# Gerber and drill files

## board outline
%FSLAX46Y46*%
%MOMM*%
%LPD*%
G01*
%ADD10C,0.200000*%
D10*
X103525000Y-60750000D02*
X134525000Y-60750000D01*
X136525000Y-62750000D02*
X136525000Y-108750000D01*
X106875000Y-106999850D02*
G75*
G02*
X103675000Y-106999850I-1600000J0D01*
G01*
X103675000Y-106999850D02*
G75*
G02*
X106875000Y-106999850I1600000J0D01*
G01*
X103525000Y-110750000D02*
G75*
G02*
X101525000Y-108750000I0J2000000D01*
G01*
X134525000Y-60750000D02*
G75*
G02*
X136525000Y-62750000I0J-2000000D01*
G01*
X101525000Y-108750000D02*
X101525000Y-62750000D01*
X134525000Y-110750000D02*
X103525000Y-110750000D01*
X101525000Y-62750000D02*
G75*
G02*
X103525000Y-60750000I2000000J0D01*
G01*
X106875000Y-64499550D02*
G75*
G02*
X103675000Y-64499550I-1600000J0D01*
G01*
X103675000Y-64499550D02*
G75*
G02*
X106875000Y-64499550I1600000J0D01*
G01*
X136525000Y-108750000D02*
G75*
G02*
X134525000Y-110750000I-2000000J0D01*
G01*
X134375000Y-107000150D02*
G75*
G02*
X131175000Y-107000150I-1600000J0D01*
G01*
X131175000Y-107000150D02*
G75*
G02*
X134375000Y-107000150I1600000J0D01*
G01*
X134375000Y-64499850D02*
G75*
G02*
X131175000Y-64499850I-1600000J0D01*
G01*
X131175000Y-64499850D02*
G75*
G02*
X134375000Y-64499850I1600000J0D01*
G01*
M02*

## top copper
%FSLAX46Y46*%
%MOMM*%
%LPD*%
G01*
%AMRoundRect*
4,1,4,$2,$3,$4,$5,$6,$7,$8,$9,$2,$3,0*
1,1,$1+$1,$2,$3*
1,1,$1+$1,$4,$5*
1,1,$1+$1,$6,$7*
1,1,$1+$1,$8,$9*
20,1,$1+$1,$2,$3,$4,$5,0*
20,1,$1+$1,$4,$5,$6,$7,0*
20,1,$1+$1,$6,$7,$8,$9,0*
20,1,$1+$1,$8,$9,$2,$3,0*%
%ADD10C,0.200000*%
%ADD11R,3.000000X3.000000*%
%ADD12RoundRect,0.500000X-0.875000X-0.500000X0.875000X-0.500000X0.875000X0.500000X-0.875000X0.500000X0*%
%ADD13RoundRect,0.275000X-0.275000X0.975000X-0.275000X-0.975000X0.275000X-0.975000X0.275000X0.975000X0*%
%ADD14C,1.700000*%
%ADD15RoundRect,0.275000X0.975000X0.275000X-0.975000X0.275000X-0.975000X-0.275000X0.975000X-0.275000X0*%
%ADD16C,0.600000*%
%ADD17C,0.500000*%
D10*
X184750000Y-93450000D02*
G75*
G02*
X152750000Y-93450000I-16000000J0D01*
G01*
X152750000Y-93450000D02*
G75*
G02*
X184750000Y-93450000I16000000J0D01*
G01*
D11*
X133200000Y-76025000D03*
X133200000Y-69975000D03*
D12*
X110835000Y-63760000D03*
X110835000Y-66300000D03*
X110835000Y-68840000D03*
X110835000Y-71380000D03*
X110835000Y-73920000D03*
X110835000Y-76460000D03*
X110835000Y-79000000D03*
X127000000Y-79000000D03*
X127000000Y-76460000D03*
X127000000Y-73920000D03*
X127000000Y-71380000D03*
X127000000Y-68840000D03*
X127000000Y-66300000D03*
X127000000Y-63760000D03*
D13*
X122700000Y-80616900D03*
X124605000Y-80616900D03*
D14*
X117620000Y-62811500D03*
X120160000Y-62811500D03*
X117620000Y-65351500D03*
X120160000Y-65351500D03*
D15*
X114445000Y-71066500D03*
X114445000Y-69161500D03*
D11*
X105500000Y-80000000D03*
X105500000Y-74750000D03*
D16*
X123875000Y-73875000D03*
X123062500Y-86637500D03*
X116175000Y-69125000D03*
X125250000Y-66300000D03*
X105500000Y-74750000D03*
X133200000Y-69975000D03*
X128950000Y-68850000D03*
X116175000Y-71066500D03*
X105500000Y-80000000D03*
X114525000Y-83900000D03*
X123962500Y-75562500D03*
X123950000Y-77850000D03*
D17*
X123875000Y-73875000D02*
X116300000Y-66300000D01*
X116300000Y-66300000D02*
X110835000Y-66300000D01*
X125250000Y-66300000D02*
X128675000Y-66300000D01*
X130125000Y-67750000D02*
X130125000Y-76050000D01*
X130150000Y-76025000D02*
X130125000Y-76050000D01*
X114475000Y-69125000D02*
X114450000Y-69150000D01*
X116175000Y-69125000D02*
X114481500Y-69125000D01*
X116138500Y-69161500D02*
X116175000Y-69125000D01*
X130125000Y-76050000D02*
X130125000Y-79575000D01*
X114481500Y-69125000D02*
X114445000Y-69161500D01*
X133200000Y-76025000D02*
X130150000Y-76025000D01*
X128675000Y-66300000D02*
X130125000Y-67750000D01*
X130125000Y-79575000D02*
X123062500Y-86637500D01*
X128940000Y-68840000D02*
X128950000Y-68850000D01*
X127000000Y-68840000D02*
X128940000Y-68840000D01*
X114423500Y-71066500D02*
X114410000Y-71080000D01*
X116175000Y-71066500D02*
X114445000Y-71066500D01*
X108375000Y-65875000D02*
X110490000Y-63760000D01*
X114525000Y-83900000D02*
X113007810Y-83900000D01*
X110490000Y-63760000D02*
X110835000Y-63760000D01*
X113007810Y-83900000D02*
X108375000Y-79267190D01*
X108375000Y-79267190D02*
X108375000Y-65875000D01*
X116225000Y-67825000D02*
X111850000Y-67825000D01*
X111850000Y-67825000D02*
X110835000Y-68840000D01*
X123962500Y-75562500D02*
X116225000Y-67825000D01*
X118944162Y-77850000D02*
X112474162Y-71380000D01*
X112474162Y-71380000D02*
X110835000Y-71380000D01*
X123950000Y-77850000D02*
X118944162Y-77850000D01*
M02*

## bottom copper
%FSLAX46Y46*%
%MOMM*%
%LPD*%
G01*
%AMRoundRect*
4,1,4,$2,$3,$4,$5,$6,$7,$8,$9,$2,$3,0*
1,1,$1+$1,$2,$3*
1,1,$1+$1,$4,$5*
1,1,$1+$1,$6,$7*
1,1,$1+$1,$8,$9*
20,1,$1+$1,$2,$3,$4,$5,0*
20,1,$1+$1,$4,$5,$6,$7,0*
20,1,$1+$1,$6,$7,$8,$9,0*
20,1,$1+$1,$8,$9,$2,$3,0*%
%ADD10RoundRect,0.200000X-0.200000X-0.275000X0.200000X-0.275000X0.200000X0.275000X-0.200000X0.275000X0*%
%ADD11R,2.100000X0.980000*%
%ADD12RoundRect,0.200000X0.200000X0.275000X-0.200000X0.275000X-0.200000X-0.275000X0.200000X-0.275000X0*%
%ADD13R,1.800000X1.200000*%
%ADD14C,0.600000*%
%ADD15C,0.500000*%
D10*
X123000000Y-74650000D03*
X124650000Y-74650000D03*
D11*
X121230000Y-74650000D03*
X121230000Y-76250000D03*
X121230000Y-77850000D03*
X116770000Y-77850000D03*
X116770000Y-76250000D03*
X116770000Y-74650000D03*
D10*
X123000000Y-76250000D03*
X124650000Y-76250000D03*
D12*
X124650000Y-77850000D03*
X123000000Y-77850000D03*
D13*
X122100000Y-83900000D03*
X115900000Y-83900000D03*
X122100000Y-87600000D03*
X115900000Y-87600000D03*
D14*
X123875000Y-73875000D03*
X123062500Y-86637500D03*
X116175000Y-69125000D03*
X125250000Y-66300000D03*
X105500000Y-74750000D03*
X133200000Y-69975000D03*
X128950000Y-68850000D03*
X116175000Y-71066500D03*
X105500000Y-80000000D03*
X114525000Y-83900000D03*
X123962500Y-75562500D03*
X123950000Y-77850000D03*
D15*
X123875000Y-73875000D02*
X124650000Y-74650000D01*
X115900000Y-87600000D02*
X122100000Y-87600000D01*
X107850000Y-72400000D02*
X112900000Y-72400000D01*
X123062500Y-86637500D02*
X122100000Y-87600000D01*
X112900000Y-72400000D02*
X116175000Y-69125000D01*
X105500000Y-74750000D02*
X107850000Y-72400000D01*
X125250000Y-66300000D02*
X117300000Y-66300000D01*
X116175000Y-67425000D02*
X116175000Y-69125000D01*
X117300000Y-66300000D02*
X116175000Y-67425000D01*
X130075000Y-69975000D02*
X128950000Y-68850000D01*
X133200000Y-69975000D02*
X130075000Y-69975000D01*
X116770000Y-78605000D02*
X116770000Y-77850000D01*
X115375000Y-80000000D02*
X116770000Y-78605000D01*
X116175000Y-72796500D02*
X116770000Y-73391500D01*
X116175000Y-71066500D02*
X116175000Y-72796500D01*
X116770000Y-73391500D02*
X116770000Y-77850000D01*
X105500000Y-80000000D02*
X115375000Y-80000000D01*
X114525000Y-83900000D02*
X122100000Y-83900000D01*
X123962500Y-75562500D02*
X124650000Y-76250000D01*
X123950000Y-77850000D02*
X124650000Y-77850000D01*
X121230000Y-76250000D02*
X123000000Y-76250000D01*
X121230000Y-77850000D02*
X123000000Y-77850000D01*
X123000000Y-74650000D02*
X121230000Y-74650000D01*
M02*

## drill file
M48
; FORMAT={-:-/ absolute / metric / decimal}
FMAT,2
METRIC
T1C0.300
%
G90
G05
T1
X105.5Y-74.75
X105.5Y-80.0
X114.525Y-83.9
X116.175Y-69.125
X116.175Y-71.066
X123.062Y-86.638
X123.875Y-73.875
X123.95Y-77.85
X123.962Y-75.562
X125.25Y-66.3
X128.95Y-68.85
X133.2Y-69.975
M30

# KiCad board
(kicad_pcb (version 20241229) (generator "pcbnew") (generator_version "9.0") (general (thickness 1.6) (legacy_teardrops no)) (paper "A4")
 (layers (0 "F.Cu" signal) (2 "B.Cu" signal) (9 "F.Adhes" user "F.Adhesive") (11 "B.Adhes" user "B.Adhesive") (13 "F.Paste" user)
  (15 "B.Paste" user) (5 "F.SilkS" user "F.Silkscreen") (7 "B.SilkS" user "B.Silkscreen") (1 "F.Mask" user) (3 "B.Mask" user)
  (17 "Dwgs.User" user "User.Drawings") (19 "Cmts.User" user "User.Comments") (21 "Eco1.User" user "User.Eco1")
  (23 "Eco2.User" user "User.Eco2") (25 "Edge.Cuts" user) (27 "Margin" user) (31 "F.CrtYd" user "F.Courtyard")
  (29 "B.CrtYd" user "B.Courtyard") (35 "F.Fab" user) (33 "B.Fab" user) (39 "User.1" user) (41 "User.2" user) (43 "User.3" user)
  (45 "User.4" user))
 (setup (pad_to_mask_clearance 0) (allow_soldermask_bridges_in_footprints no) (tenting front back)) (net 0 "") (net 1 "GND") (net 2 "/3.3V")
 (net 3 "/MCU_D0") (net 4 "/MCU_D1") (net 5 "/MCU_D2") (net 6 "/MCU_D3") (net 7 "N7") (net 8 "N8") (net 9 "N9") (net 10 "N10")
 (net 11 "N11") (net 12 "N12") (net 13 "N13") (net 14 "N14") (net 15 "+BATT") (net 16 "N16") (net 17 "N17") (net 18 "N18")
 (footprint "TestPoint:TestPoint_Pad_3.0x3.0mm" (layer "F.Cu") (at 133.2 76.025)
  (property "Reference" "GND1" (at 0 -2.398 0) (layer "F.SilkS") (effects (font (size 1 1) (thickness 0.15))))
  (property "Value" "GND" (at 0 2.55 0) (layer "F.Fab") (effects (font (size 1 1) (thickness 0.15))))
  (pad "1" smd rect (at 0 0) (size 3 3) (layers "F.Cu" "F.Mask") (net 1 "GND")))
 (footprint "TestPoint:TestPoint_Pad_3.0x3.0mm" (layer "F.Cu") (at 133.2 69.975)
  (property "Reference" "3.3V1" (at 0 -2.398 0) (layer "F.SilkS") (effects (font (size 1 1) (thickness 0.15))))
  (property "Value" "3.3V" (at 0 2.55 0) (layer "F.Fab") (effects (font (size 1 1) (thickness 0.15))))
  (pad "1" smd rect (at 0 0) (size 3 3) (layers "F.Cu" "F.Mask") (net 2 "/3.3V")))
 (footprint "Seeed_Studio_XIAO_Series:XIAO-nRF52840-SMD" (layer "F.Cu") (at 110 81.88)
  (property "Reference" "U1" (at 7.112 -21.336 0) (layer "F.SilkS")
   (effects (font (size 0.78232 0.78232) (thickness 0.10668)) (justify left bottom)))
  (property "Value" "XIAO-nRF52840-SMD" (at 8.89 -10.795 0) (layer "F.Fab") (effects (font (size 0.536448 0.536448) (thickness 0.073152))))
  (pad "1" smd roundrect (at 0.835 -18.12) (size 2.75 2) (layers "F.Cu" "F.Mask" "F.Paste") (roundrect_rratio 0.25) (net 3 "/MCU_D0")
   (solder_mask_margin 0.0508) (thermal_bridge_angle 45))
  (pad "2" smd roundrect (at 0.835 -15.58) (size 2.75 2) (layers "F.Cu" "F.Mask" "F.Paste") (roundrect_rratio 0.25) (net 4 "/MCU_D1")
   (solder_mask_margin 0.0508) (thermal_bridge_angle 45))
  (pad "3" smd roundrect (at 0.835 -13.04) (size 2.75 2) (layers "F.Cu" "F.Mask" "F.Paste") (roundrect_rratio 0.25) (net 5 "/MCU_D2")
   (solder_mask_margin 0.0508) (thermal_bridge_angle 45))
  (pad "4" smd roundrect (at 0.835 -10.5) (size 2.75 2) (layers "F.Cu" "F.Mask" "F.Paste") (roundrect_rratio 0.25) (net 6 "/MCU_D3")
   (solder_mask_margin 0.0508) (thermal_bridge_angle 45))
  (pad "5" smd roundrect (at 0.835 -7.96) (size 2.75 2) (layers "F.Cu" "F.Mask" "F.Paste") (roundrect_rratio 0.25) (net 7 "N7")
   (solder_mask_margin 0.0508) (thermal_bridge_angle 45))
  (pad "6" smd roundrect (at 0.835 -5.42) (size 2.75 2) (layers "F.Cu" "F.Mask" "F.Paste") (roundrect_rratio 0.25) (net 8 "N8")
   (solder_mask_margin 0.0508) (thermal_bridge_angle 45))
  (pad "7" smd roundrect (at 0.835 -2.88) (size 2.75 2) (layers "F.Cu" "F.Mask" "F.Paste") (roundrect_rratio 0.25) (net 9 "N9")
   (solder_mask_margin 0.0508) (thermal_bridge_angle 45))
  (pad "8" smd roundrect (at 17 -2.88) (size 2.75 2) (layers "F.Cu" "F.Mask" "F.Paste") (roundrect_rratio 0.25) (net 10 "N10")
   (solder_mask_margin 0.0508) (thermal_bridge_angle 45))
  (pad "9" smd roundrect (at 17 -5.42) (size 2.75 2) (layers "F.Cu" "F.Mask" "F.Paste") (roundrect_rratio 0.25) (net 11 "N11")
   (solder_mask_margin 0.0508) (thermal_bridge_angle 45))
  (pad "10" smd roundrect (at 17 -7.96) (size 2.75 2) (layers "F.Cu" "F.Mask" "F.Paste") (roundrect_rratio 0.25) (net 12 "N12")
   (solder_mask_margin 0.0508) (thermal_bridge_angle 45))
  (pad "11" smd roundrect (at 17 -10.5) (size 2.75 2) (layers "F.Cu" "F.Mask" "F.Paste") (roundrect_rratio 0.25) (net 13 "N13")
   (solder_mask_margin 0.0508) (thermal_bridge_angle 45))
  (pad "12" smd roundrect (at 17 -13.04) (size 2.75 2) (layers "F.Cu" "F.Mask" "F.Paste") (roundrect_rratio 0.25) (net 2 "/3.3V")
   (solder_mask_margin 0.0508) (thermal_bridge_angle 45))
  (pad "13" smd roundrect (at 17 -15.58) (size 2.75 2) (layers "F.Cu" "F.Mask" "F.Paste") (roundrect_rratio 0.25) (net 1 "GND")
   (solder_mask_margin 0.0508) (thermal_bridge_angle 45))
  (pad "14" smd roundrect (at 17 -18.12) (size 2.75 2) (layers "F.Cu" "F.Mask" "F.Paste") (roundrect_rratio 0.25) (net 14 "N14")
   (solder_mask_margin 0.0508) (thermal_bridge_angle 45))
  (pad "17" smd roundrect (at 12.7 -1.2631 270) (size 2.5 1.1) (layers "F.Cu" "F.Mask" "F.Paste") (roundrect_rratio 0.25)
   (solder_mask_margin 0.0508) (thermal_bridge_angle 45))
  (pad "18" smd roundrect (at 14.605 -1.2631 270) (size 2.5 1.1) (layers "F.Cu" "F.Mask" "F.Paste") (roundrect_rratio 0.25)
   (solder_mask_margin 0.0508) (thermal_bridge_angle 45))
  (pad "19" smd circle (at 7.62 -19.0685) (size 1.7 1.7) (layers "F.Cu" "F.Mask" "F.Paste"))
  (pad "20" smd circle (at 10.16 -19.0685) (size 1.7 1.7) (layers "F.Cu" "F.Mask" "F.Paste"))
  (pad "21" smd circle (at 7.62 -16.5285) (size 1.7 1.7) (layers "F.Cu" "F.Mask" "F.Paste"))
  (pad "22" smd circle (at 10.16 -16.5285) (size 1.7 1.7) (layers "F.Cu" "F.Mask" "F.Paste"))
  (pad "32" smd roundrect (at 4.445 -10.8135 180) (size 2.5 1.1) (layers "F.Cu" "F.Mask" "F.Paste") (roundrect_rratio 0.25) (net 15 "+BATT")
   (solder_mask_margin 0.0508) (thermal_bridge_angle 45))
  (pad "33" smd roundrect (at 4.445 -12.7185 180) (size 2.5 1.1) (layers "F.Cu" "F.Mask" "F.Paste") (roundrect_rratio 0.25) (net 1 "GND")
   (solder_mask_margin 0.0508) (thermal_bridge_angle 45)))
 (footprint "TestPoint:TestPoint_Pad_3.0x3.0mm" (layer "F.Cu") (at 105.5 80 90)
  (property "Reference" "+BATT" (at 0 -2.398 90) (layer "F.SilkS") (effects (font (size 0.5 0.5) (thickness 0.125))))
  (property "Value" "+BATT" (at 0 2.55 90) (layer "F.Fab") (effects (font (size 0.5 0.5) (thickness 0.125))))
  (pad "1" smd rect (at 0 0 90) (size 3 3) (layers "F.Cu" "F.Mask") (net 15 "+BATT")))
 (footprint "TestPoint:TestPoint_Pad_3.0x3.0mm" (layer "F.Cu") (at 105.5 74.75 90)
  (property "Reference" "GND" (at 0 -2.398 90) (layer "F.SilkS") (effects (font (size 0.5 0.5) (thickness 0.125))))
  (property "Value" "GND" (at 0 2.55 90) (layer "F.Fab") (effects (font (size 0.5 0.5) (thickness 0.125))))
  (pad "1" smd rect (at 0 0 90) (size 3 3) (layers "F.Cu" "F.Mask") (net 1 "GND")))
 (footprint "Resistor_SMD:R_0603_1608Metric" (layer "B.Cu") (at 123.825 74.65)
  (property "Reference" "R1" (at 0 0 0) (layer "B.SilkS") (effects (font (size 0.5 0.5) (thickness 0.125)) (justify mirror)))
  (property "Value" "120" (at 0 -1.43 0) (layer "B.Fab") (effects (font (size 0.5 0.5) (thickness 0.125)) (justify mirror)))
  (pad "1" smd roundrect (at -0.825 0) (size 0.8 0.95) (layers "B.Cu" "B.Mask" "B.Paste") (roundrect_rratio 0.25) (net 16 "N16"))
  (pad "2" smd roundrect (at 0.825 0) (size 0.8 0.95) (layers "B.Cu" "B.Mask" "B.Paste") (roundrect_rratio 0.25) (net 4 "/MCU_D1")))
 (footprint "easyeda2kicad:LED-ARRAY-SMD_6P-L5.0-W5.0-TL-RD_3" (layer "B.Cu") (at 119 76.25 180)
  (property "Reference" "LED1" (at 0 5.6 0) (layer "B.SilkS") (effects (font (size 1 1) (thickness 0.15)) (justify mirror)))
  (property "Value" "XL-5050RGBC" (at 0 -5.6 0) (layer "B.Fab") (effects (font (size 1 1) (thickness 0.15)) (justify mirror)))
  (pad "1" smd rect (at -2.23 1.6 180) (size 2.1 0.98) (layers "B.Cu" "B.Mask" "B.Paste") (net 16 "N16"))
  (pad "2" smd rect (at -2.23 0 180) (size 2.1 0.98) (layers "B.Cu" "B.Mask" "B.Paste") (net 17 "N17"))
  (pad "3" smd rect (at -2.23 -1.6 180) (size 2.1 0.98) (layers "B.Cu" "B.Mask" "B.Paste") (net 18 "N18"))
  (pad "4" smd rect (at 2.23 -1.6 180) (size 2.1 0.98) (layers "B.Cu" "B.Mask" "B.Paste") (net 15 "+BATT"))
  (pad "5" smd rect (at 2.23 0 180) (size 2.1 0.98) (layers "B.Cu" "B.Mask" "B.Paste") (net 15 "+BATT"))
  (pad "6" smd rect (at 2.23 1.6 180) (size 2.1 0.98) (layers "B.Cu" "B.Mask" "B.Paste") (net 15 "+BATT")))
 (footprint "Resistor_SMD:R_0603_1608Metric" (layer "B.Cu") (at 123.825 76.25)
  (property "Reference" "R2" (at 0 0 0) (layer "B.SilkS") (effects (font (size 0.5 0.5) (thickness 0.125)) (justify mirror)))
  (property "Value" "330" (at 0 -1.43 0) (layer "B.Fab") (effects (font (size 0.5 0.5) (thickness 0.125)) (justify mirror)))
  (pad "1" smd roundrect (at -0.825 0) (size 0.8 0.95) (layers "B.Cu" "B.Mask" "B.Paste") (roundrect_rratio 0.25) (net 17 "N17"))
  (pad "2" smd roundrect (at 0.825 0) (size 0.8 0.95) (layers "B.Cu" "B.Mask" "B.Paste") (roundrect_rratio 0.25) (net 5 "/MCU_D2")))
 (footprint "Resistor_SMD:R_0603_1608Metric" (layer "B.Cu") (at 123.825 77.85 180)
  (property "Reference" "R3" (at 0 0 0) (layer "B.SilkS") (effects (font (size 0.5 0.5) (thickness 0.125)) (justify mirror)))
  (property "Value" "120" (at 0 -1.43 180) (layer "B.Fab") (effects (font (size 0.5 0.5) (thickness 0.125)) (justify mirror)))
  (pad "1" smd roundrect (at -0.825 0 180) (size 0.8 0.95) (layers "B.Cu" "B.Mask" "B.Paste") (roundrect_rratio 0.25) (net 6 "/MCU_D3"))
  (pad "2" smd roundrect (at 0.825 0 180) (size 0.8 0.95) (layers "B.Cu" "B.Mask" "B.Paste") (roundrect_rratio 0.25) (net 18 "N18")))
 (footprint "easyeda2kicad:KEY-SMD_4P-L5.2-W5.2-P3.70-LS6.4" (layer "B.Cu") (at 119 85.75 180)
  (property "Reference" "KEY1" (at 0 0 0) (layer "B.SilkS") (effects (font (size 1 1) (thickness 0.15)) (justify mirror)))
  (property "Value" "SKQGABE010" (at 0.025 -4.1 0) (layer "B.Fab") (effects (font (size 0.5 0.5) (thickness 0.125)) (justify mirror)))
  (pad "1" smd rect (at -3.1 1.85 180) (size 1.8 1.2) (layers "B.Cu" "B.Mask" "B.Paste") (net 3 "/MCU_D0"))
  (pad "2" smd rect (at 3.1 1.85 180) (size 1.8 1.2) (layers "B.Cu" "B.Mask" "B.Paste") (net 3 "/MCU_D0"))
  (pad "3" smd rect (at -3.1 -1.85 180) (size 1.8 1.2) (layers "B.Cu" "B.Mask" "B.Paste") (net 1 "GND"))
  (pad "4" smd rect (at 3.1 -1.85 180) (size 1.8 1.2) (layers "B.Cu" "B.Mask" "B.Paste") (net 1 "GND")))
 (gr_circle (center 168.75 93.45) (end 184.75 93.45) (stroke (width 0.2) (type solid)) (fill no) (layer "F.Cu"))
 (gr_line (start 103.525 60.75) (end 134.525 60.75) (stroke (width 0.2) (type default)) (layer "Edge.Cuts"))
 (gr_line (start 136.525 62.75) (end 136.525 108.75) (stroke (width 0.2) (type default)) (layer "Edge.Cuts"))
 (gr_circle (center 105.275 106.99985) (end 106.875 106.99985) (stroke (width 0.2) (type solid)) (fill no) (layer "Edge.Cuts"))
 (gr_arc (start 103.525 110.75) (mid 102.110786 110.164214) (end 101.525 108.75) (stroke (width 0.2) (type default)) (layer "Edge.Cuts"))
 (gr_arc (start 134.525 60.75) (mid 135.939214 61.335786) (end 136.525 62.75) (stroke (width 0.2) (type default)) (layer "Edge.Cuts"))
 (gr_line (start 101.525 108.75) (end 101.525 62.75) (stroke (width 0.2) (type default)) (layer "Edge.Cuts"))
 (gr_line (start 134.525 110.75) (end 103.525 110.75) (stroke (width 0.2) (type default)) (layer "Edge.Cuts"))
 (gr_arc (start 101.525 62.75) (mid 102.110786 61.335786) (end 103.525 60.75) (stroke (width 0.2) (type default)) (layer "Edge.Cuts"))
 (gr_circle (center 105.275 64.49955) (end 106.875 64.49955) (stroke (width 0.2) (type solid)) (fill no) (layer "Edge.Cuts"))
 (gr_arc (start 136.525 108.75) (mid 135.939214 110.164214) (end 134.525 110.75) (stroke (width 0.2) (type default)) (layer "Edge.Cuts"))
 (gr_circle (center 132.775 107.00015) (end 134.375 107.00015) (stroke (width 0.2) (type solid)) (fill no) (layer "Edge.Cuts"))
 (gr_circle (center 132.775 64.49985) (end 134.375 64.49985) (stroke (width 0.2) (type solid)) (fill no) (layer "Edge.Cuts"))
 (segment (start 123.875 73.875) (end 116.3 66.3) (width 0.5) (layer "F.Cu") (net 4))
 (segment (start 116.3 66.3) (end 110.835 66.3) (width 0.5) (layer "F.Cu") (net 4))
 (via (at 123.875 73.875) (size 0.6) (drill 0.3) (layers "F.Cu" "B.Cu") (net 4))
 (segment (start 123.875 73.875) (end 124.65 74.65) (width 0.5) (layer "B.Cu") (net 4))
 (segment (start 125.25 66.3) (end 128.675 66.3) (width 0.5) (layer "F.Cu") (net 1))
 (segment (start 130.125 67.75) (end 130.125 76.05) (width 0.5) (layer "F.Cu") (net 1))
 (segment (start 130.15 76.025) (end 130.125 76.05) (width 0.5) (layer "F.Cu") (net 1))
 (segment (start 114.475 69.125) (end 114.45 69.15) (width 0.5) (layer "F.Cu") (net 1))
 (segment (start 116.175 69.125) (end 114.4815 69.125) (width 0.5) (layer "F.Cu") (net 1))
 (segment (start 116.1385 69.1615) (end 116.175 69.125) (width 0.5) (layer "F.Cu") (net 1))
 (segment (start 130.125 76.05) (end 130.125 79.575) (width 0.5) (layer "F.Cu") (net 1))
 (segment (start 114.4815 69.125) (end 114.445 69.1615) (width 0.5) (layer "F.Cu") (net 1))
 (segment (start 133.2 76.025) (end 130.15 76.025) (width 0.5) (layer "F.Cu") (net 1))
 (segment (start 128.675 66.3) (end 130.125 67.75) (width 0.5) (layer "F.Cu") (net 1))
 (segment (start 130.125 79.575) (end 123.0625 86.6375) (width 0.5) (layer "F.Cu") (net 1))
 (via (at 123.0625 86.6375) (size 0.6) (drill 0.3) (layers "F.Cu" "B.Cu") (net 1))
 (via (at 116.175 69.125) (size 0.6) (drill 0.3) (layers "F.Cu" "B.Cu") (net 1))
 (via (at 125.25 66.3) (size 0.6) (drill 0.3) (layers "F.Cu" "B.Cu") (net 1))
 (via (at 105.5 74.75) (size 0.6) (drill 0.3) (layers "F.Cu" "B.Cu") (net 1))
 (segment (start 115.9 87.6) (end 122.1 87.6) (width 0.5) (layer "B.Cu") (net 1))
 (segment (start 107.85 72.4) (end 112.9 72.4) (width 0.5) (layer "B.Cu") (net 1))
 (segment (start 123.0625 86.6375) (end 122.1 87.6) (width 0.5) (layer "B.Cu") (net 1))
 (segment (start 112.9 72.4) (end 116.175 69.125) (width 0.5) (layer "B.Cu") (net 1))
 (segment (start 105.5 74.75) (end 107.85 72.4) (width 0.5) (layer "B.Cu") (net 1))
 (segment (start 125.25 66.3) (end 117.3 66.3) (width 0.5) (layer "B.Cu") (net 1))
 (segment (start 116.175 67.425) (end 116.175 69.125) (width 0.5) (layer "B.Cu") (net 1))
 (segment (start 117.3 66.3) (end 116.175 67.425) (width 0.5) (layer "B.Cu") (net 1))
 (segment (start 128.94 68.84) (end 128.95 68.85) (width 0.5) (layer "F.Cu") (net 2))
 (segment (start 127 68.84) (end 128.94 68.84) (width 0.5) (layer "F.Cu") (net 2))
 (via (at 133.2 69.975) (size 0.6) (drill 0.3) (layers "F.Cu" "B.Cu") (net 2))
 (via (at 128.95 68.85) (size 0.6) (drill 0.3) (layers "F.Cu" "B.Cu") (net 2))
 (segment (start 130.075 69.975) (end 128.95 68.85) (width 0.5) (layer "B.Cu") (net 2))
 (segment (start 133.2 69.975) (end 130.075 69.975) (width 0.5) (layer "B.Cu") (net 2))
 (segment (start 114.4235 71.0665) (end 114.41 71.08) (width 0.5) (layer "F.Cu") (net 15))
 (segment (start 116.175 71.0665) (end 114.445 71.0665) (width 0.5) (layer "F.Cu") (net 15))
 (via (at 116.175 71.0665) (size 0.6) (drill 0.3) (layers "F.Cu" "B.Cu") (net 15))
 (via (at 105.5 80) (size 0.6) (drill 0.3) (layers "F.Cu" "B.Cu") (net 15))
 (segment (start 116.77 78.605) (end 116.77 77.85) (width 0.5) (layer "B.Cu") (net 15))
 (segment (start 115.375 80) (end 116.77 78.605) (width 0.5) (layer "B.Cu") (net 15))
 (segment (start 116.175 72.7965) (end 116.77 73.3915) (width 0.5) (layer "B.Cu") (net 15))
 (segment (start 116.175 71.0665) (end 116.175 72.7965) (width 0.5) (layer "B.Cu") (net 15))
 (segment (start 116.77 73.3915) (end 116.77 77.85) (width 0.5) (layer "B.Cu") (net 15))
 (segment (start 105.5 80) (end 115.375 80) (width 0.5) (layer "B.Cu") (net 15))
 (segment (start 108.375 65.875) (end 110.49 63.76) (width 0.5) (layer "F.Cu") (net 3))
 (segment (start 114.525 83.9) (end 113.00781 83.9) (width 0.5) (layer "F.Cu") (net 3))
 (segment (start 110.49 63.76) (end 110.835 63.76) (width 0.5) (layer "F.Cu") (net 3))
 (segment (start 113.00781 83.9) (end 108.375 79.26719) (width 0.5) (layer "F.Cu") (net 3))
 (segment (start 108.375 79.26719) (end 108.375 65.875) (width 0.5) (layer "F.Cu") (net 3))
 (via (at 114.525 83.9) (size 0.6) (drill 0.3) (layers "F.Cu" "B.Cu") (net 3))
 (segment (start 114.525 83.9) (end 122.1 83.9) (width 0.5) (layer "B.Cu") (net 3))
 (segment (start 116.225 67.825) (end 111.85 67.825) (width 0.5) (layer "F.Cu") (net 5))
 (segment (start 111.85 67.825) (end 110.835 68.84) (width 0.5) (layer "F.Cu") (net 5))
 (segment (start 123.9625 75.5625) (end 116.225 67.825) (width 0.5) (layer "F.Cu") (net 5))
 (via (at 123.9625 75.5625) (size 0.6) (drill 0.3) (layers "F.Cu" "B.Cu") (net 5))
 (segment (start 123.9625 75.5625) (end 124.65 76.25) (width 0.5) (layer "B.Cu") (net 5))
 (segment (start 118.944162 77.85) (end 112.474162 71.38) (width 0.5) (layer "F.Cu") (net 6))
 (segment (start 112.474162 71.38) (end 110.835 71.38) (width 0.5) (layer "F.Cu") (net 6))
 (segment (start 123.95 77.85) (end 118.944162 77.85) (width 0.5) (layer "F.Cu") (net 6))
 (via (at 123.95 77.85) (size 0.6) (drill 0.3) (layers "F.Cu" "B.Cu") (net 6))
 (segment (start 123.95 77.85) (end 124.65 77.85) (width 0.5) (layer "B.Cu") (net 6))
 (segment (start 121.23 76.25) (end 123 76.25) (width 0.5) (layer "B.Cu") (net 17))
 (segment (start 121.23 77.85) (end 123 77.85) (width 0.5) (layer "B.Cu") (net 18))
 (segment (start 123 74.65) (end 121.23 74.65) (width 0.5) (layer "B.Cu") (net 16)))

